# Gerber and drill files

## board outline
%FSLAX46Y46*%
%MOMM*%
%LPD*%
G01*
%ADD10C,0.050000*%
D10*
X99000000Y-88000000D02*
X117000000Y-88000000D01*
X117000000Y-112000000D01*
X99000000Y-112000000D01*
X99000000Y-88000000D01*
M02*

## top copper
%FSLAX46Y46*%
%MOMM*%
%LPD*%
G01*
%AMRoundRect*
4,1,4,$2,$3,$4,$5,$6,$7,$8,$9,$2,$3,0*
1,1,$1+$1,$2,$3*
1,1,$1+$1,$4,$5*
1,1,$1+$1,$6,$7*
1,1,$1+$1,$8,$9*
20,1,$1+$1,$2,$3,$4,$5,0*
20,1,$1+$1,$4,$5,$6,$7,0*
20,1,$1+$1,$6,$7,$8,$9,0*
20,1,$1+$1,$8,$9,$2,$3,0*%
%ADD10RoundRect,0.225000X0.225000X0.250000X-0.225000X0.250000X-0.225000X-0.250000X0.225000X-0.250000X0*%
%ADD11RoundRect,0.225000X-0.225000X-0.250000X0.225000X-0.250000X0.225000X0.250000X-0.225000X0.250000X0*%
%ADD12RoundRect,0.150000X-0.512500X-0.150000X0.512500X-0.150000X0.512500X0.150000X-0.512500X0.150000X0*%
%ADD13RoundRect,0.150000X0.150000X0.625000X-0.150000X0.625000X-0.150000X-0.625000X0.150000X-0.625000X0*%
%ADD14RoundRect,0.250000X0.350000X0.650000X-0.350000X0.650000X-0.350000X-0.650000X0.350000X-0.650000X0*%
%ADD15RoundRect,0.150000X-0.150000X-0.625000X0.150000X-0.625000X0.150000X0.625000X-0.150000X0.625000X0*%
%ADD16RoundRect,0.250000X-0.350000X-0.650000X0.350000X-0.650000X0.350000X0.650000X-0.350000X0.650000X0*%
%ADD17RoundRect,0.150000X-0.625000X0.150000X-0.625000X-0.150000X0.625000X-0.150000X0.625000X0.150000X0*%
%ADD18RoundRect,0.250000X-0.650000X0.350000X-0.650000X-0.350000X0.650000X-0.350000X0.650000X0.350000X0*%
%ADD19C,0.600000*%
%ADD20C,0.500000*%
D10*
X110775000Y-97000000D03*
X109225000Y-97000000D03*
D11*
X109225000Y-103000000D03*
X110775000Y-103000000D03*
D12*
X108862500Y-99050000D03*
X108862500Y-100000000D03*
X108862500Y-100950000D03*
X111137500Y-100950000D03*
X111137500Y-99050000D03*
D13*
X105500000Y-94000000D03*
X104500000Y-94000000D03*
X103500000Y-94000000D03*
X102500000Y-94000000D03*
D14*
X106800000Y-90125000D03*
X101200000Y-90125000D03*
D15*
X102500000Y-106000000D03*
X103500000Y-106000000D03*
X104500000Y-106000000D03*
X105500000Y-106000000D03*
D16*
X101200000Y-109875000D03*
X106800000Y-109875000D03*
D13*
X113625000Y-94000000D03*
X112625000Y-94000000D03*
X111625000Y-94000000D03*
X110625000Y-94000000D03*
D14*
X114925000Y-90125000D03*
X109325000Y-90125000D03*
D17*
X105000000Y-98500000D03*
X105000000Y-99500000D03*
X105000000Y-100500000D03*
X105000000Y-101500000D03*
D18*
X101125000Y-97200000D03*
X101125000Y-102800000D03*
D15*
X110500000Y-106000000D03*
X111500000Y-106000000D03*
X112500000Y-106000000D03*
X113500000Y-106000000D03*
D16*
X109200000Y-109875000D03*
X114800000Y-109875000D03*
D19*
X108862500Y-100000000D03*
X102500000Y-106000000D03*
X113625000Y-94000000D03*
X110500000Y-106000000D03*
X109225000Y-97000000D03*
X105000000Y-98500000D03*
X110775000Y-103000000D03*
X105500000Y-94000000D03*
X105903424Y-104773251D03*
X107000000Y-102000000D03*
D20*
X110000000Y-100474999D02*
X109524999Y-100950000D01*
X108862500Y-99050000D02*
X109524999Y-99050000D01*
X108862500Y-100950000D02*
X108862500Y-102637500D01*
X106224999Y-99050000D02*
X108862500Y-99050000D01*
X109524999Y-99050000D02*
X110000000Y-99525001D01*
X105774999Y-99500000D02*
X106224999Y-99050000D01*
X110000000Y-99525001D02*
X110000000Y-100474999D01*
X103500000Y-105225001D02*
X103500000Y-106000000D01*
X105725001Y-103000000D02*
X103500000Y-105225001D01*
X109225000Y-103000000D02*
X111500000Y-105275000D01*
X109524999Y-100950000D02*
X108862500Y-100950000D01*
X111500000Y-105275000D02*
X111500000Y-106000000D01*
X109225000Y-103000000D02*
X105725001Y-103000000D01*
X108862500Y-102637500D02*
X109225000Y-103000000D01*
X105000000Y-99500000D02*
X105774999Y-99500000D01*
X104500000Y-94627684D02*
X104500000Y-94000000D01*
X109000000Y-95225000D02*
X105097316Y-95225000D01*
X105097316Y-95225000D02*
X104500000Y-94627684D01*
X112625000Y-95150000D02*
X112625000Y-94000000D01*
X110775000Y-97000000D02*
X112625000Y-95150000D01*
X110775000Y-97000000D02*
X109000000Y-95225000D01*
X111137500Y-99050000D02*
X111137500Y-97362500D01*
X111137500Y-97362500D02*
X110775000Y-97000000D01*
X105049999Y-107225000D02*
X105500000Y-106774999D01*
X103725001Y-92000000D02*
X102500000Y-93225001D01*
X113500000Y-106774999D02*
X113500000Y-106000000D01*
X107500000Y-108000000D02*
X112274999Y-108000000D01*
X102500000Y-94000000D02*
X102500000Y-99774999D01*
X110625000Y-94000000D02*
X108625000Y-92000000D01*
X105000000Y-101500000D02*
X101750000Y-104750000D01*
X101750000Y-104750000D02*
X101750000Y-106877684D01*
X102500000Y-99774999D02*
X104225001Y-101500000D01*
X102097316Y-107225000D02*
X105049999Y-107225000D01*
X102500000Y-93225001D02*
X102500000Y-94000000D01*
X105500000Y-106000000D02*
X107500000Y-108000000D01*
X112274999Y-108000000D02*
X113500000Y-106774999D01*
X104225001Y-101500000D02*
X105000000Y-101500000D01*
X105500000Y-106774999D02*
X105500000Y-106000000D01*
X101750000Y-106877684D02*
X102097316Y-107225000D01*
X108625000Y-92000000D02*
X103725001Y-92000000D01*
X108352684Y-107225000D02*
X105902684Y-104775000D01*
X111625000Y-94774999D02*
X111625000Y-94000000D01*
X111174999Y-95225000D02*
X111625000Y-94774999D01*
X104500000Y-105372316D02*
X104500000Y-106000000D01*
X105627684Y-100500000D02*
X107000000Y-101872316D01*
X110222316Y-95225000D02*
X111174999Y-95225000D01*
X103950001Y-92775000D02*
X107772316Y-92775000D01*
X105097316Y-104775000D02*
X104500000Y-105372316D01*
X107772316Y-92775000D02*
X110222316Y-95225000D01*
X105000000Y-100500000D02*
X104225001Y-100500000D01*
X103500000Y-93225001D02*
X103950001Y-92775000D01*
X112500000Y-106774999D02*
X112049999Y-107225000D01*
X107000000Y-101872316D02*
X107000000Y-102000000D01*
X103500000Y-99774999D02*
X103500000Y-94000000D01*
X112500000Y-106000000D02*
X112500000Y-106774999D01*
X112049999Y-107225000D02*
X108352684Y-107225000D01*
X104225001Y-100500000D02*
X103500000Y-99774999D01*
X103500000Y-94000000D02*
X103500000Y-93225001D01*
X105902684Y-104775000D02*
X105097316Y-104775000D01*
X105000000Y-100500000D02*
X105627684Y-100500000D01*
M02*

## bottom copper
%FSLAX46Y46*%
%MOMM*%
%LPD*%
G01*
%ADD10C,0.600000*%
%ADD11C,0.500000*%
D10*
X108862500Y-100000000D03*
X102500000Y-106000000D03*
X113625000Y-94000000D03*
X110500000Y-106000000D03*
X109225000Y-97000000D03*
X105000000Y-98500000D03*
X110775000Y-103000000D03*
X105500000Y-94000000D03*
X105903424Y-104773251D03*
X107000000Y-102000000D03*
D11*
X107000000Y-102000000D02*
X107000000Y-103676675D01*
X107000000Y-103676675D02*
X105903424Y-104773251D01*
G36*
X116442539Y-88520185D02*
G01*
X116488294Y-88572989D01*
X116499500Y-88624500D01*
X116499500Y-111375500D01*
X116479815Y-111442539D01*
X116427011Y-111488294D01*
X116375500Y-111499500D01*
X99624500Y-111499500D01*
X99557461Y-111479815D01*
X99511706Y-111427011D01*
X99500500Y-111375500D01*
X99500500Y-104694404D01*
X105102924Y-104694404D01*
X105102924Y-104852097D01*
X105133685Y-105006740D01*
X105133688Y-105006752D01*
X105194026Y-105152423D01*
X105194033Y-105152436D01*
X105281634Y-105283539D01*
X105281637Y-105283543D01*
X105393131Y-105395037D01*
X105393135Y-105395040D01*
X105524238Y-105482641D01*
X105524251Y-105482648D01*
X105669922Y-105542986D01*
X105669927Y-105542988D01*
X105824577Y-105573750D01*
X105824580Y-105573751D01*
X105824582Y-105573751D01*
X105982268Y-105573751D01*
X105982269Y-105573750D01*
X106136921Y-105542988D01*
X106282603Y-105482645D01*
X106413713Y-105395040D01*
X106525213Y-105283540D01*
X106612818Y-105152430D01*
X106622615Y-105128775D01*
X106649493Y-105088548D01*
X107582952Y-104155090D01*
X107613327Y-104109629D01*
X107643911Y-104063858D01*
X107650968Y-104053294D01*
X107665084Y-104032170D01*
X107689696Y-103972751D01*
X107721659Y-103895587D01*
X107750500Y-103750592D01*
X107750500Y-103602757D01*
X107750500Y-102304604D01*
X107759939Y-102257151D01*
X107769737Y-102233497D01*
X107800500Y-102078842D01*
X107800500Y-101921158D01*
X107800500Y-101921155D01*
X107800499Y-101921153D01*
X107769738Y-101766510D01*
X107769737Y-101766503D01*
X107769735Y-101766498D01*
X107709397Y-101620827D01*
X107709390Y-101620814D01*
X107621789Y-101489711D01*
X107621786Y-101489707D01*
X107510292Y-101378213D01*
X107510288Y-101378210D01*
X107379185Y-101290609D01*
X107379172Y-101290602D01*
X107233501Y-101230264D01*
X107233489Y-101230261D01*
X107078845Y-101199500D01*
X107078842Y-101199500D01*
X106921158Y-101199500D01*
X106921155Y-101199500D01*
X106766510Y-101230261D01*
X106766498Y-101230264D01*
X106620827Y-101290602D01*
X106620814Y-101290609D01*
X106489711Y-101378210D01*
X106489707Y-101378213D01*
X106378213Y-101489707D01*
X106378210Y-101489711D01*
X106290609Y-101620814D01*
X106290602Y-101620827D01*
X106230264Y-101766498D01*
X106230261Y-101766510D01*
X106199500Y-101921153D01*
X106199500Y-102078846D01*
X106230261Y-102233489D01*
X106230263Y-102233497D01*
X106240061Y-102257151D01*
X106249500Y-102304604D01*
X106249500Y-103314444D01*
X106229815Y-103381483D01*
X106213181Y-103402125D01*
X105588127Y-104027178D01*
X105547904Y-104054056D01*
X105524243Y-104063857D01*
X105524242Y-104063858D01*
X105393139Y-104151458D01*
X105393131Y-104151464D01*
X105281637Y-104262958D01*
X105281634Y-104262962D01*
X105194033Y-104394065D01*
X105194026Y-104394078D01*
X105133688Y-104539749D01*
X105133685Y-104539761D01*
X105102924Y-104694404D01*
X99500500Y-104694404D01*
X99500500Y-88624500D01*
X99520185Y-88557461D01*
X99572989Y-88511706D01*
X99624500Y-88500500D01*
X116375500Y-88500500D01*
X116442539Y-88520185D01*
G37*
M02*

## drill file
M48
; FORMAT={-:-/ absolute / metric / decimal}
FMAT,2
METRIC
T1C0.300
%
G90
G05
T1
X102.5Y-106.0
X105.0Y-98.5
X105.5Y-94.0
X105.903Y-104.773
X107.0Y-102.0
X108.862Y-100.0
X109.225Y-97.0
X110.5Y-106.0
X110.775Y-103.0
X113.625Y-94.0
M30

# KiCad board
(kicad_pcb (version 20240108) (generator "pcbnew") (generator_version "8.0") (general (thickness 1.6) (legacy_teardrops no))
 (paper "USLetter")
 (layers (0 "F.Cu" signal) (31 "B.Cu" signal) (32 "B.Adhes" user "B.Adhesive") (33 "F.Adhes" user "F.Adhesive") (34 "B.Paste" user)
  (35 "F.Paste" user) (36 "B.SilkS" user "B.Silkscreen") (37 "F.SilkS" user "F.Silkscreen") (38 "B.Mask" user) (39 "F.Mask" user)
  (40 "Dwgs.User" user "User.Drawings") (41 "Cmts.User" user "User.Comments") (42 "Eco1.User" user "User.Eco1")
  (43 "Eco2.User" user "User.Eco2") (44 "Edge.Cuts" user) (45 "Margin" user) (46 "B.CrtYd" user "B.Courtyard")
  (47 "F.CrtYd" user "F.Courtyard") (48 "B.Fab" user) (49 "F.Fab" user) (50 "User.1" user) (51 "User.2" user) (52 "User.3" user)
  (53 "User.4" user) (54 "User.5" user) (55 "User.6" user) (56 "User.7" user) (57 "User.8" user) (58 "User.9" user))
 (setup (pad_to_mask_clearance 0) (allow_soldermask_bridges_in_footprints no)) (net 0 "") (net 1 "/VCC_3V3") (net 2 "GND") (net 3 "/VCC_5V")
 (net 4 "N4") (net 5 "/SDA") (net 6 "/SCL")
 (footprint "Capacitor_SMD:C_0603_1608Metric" (layer "F.Cu") (at 110 97 180)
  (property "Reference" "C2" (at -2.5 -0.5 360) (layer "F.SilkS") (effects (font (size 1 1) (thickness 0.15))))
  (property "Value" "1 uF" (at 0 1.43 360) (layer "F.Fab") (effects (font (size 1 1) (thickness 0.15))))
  (pad "1" smd roundrect (at -0.775 0 180) (size 0.9 0.95) (layers "F.Cu" "F.Paste" "F.Mask") (roundrect_rratio 0.25) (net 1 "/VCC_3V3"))
  (pad "2" smd roundrect (at 0.775 0 180) (size 0.9 0.95) (layers "F.Cu" "F.Paste" "F.Mask") (roundrect_rratio 0.25) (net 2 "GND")))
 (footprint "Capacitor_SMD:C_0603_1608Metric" (layer "F.Cu") (at 110 103)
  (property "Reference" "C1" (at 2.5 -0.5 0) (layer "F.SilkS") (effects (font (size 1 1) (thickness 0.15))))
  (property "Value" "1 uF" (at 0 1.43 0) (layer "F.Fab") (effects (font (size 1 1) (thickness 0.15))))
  (pad "1" smd roundrect (at -0.775 0) (size 0.9 0.95) (layers "F.Cu" "F.Paste" "F.Mask") (roundrect_rratio 0.25) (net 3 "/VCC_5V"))
  (pad "2" smd roundrect (at 0.775 0) (size 0.9 0.95) (layers "F.Cu" "F.Paste" "F.Mask") (roundrect_rratio 0.25) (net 2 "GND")))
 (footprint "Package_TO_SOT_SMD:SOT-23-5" (layer "F.Cu") (at 110 100)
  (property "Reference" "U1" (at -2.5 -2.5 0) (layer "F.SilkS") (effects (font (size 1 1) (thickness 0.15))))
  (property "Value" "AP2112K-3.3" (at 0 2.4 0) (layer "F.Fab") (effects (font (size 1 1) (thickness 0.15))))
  (pad "1" smd roundrect (at -1.1375 -0.95) (size 1.325 0.6) (layers "F.Cu" "F.Paste" "F.Mask") (roundrect_rratio 0.25) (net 3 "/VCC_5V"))
  (pad "2" smd roundrect (at -1.1375 0) (size 1.325 0.6) (layers "F.Cu" "F.Paste" "F.Mask") (roundrect_rratio 0.25) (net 2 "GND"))
  (pad "3" smd roundrect (at -1.1375 0.95) (size 1.325 0.6) (layers "F.Cu" "F.Paste" "F.Mask") (roundrect_rratio 0.25) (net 3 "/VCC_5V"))
  (pad "4" smd roundrect (at 1.1375 0.95) (size 1.325 0.6) (layers "F.Cu" "F.Paste" "F.Mask") (roundrect_rratio 0.25) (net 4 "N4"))
  (pad "5" smd roundrect (at 1.1375 -0.95) (size 1.325 0.6) (layers "F.Cu" "F.Paste" "F.Mask") (roundrect_rratio 0.25) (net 1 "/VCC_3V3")))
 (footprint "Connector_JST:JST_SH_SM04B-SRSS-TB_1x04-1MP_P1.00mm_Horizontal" (layer "F.Cu") (at 104 92 180)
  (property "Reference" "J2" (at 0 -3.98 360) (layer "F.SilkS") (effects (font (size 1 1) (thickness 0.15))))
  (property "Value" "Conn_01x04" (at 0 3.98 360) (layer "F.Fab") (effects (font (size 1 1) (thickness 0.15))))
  (pad "1" smd roundrect (at -1.5 -2 180) (size 0.6 1.55) (layers "F.Cu" "F.Paste" "F.Mask") (roundrect_rratio 0.25) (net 2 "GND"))
  (pad "2" smd roundrect (at -0.5 -2 180) (size 0.6 1.55) (layers "F.Cu" "F.Paste" "F.Mask") (roundrect_rratio 0.25) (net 1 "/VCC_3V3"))
  (pad "3" smd roundrect (at 0.5 -2 180) (size 0.6 1.55) (layers "F.Cu" "F.Paste" "F.Mask") (roundrect_rratio 0.25) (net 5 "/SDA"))
  (pad "4" smd roundrect (at 1.5 -2 180) (size 0.6 1.55) (layers "F.Cu" "F.Paste" "F.Mask") (roundrect_rratio 0.25) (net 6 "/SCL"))
  (pad "MP" smd roundrect (at -2.8 1.875 180) (size 1.2 1.8) (layers "F.Cu" "F.Paste" "F.Mask") (roundrect_rratio 0.208333))
  (pad "MP" smd roundrect (at 2.8 1.875 180) (size 1.2 1.8) (layers "F.Cu" "F.Paste" "F.Mask") (roundrect_rratio 0.208333)))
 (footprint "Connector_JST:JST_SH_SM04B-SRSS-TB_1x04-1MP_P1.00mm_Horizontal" (layer "F.Cu") (at 104 108)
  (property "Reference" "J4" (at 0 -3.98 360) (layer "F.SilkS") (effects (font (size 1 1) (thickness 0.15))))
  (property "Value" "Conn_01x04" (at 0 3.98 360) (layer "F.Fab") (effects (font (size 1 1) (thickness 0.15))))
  (pad "1" smd roundrect (at -1.5 -2) (size 0.6 1.55) (layers "F.Cu" "F.Paste" "F.Mask") (roundrect_rratio 0.25) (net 2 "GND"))
  (pad "2" smd roundrect (at -0.5 -2) (size 0.6 1.55) (layers "F.Cu" "F.Paste" "F.Mask") (roundrect_rratio 0.25) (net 3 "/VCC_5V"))
  (pad "3" smd roundrect (at 0.5 -2) (size 0.6 1.55) (layers "F.Cu" "F.Paste" "F.Mask") (roundrect_rratio 0.25) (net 5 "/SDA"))
  (pad "4" smd roundrect (at 1.5 -2) (size 0.6 1.55) (layers "F.Cu" "F.Paste" "F.Mask") (roundrect_rratio 0.25) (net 6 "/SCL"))
  (pad "MP" smd roundrect (at -2.8 1.875) (size 1.2 1.8) (layers "F.Cu" "F.Paste" "F.Mask") (roundrect_rratio 0.208333))
  (pad "MP" smd roundrect (at 2.8 1.875) (size 1.2 1.8) (layers "F.Cu" "F.Paste" "F.Mask") (roundrect_rratio 0.208333)))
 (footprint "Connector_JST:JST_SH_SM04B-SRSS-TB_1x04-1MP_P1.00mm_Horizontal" (layer "F.Cu") (at 112.125 92 180)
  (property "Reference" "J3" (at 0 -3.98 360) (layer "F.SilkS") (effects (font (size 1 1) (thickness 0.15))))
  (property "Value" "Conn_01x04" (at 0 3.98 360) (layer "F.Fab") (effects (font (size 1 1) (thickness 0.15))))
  (pad "1" smd roundrect (at -1.5 -2 180) (size 0.6 1.55) (layers "F.Cu" "F.Paste" "F.Mask") (roundrect_rratio 0.25) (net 2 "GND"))
  (pad "2" smd roundrect (at -0.5 -2 180) (size 0.6 1.55) (layers "F.Cu" "F.Paste" "F.Mask") (roundrect_rratio 0.25) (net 1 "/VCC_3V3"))
  (pad "3" smd roundrect (at 0.5 -2 180) (size 0.6 1.55) (layers "F.Cu" "F.Paste" "F.Mask") (roundrect_rratio 0.25) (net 5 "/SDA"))
  (pad "4" smd roundrect (at 1.5 -2 180) (size 0.6 1.55) (layers "F.Cu" "F.Paste" "F.Mask") (roundrect_rratio 0.25) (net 6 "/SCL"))
  (pad "MP" smd roundrect (at -2.8 1.875 180) (size 1.2 1.8) (layers "F.Cu" "F.Paste" "F.Mask") (roundrect_rratio 0.208333))
  (pad "MP" smd roundrect (at 2.8 1.875 180) (size 1.2 1.8) (layers "F.Cu" "F.Paste" "F.Mask") (roundrect_rratio 0.208333)))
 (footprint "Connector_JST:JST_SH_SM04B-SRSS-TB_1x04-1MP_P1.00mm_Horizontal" (layer "F.Cu") (at 103 100 -90)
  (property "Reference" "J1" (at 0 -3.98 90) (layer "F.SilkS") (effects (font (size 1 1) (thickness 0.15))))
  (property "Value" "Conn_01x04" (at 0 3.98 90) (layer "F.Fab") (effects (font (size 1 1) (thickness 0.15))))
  (pad "1" smd roundrect (at -1.5 -2 270) (size 0.6 1.55) (layers "F.Cu" "F.Paste" "F.Mask") (roundrect_rratio 0.25) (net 2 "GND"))
  (pad "2" smd roundrect (at -0.5 -2 270) (size 0.6 1.55) (layers "F.Cu" "F.Paste" "F.Mask") (roundrect_rratio 0.25) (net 3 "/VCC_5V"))
  (pad "3" smd roundrect (at 0.5 -2 270) (size 0.6 1.55) (layers "F.Cu" "F.Paste" "F.Mask") (roundrect_rratio 0.25) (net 5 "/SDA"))
  (pad "4" smd roundrect (at 1.5 -2 270) (size 0.6 1.55) (layers "F.Cu" "F.Paste" "F.Mask") (roundrect_rratio 0.25) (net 6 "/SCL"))
  (pad "MP" smd roundrect (at -2.8 1.875 270) (size 1.2 1.8) (layers "F.Cu" "F.Paste" "F.Mask") (roundrect_rratio 0.208333))
  (pad "MP" smd roundrect (at 2.8 1.875 270) (size 1.2 1.8) (layers "F.Cu" "F.Paste" "F.Mask") (roundrect_rratio 0.208333)))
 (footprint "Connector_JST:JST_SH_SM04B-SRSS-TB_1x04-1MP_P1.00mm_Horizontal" (layer "F.Cu") (at 112 108)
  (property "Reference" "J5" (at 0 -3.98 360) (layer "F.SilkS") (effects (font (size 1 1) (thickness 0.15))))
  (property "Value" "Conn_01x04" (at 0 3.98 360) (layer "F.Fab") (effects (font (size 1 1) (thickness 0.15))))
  (pad "1" smd roundrect (at -1.5 -2) (size 0.6 1.55) (layers "F.Cu" "F.Paste" "F.Mask") (roundrect_rratio 0.25) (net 2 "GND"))
  (pad "2" smd roundrect (at -0.5 -2) (size 0.6 1.55) (layers "F.Cu" "F.Paste" "F.Mask") (roundrect_rratio 0.25) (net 3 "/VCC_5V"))
  (pad "3" smd roundrect (at 0.5 -2) (size 0.6 1.55) (layers "F.Cu" "F.Paste" "F.Mask") (roundrect_rratio 0.25) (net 5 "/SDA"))
  (pad "4" smd roundrect (at 1.5 -2) (size 0.6 1.55) (layers "F.Cu" "F.Paste" "F.Mask") (roundrect_rratio 0.25) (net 6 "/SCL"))
  (pad "MP" smd roundrect (at -2.8 1.875) (size 1.2 1.8) (layers "F.Cu" "F.Paste" "F.Mask") (roundrect_rratio 0.208333))
  (pad "MP" smd roundrect (at 2.8 1.875) (size 1.2 1.8) (layers "F.Cu" "F.Paste" "F.Mask") (roundrect_rratio 0.208333)))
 (gr_rect (start 99 88) (end 117 112) (stroke (width 0.05) (type default)) (fill none) (layer "Edge.Cuts"))
 (via (at 108.8625 100) (size 0.6) (drill 0.3) (layers "F.Cu" "B.Cu") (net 2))
 (via (at 102.5 106) (size 0.6) (drill 0.3) (layers "F.Cu" "B.Cu") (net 2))
 (via (at 113.625 94) (size 0.6) (drill 0.3) (layers "F.Cu" "B.Cu") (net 2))
 (via (at 110.5 106) (size 0.6) (drill 0.3) (layers "F.Cu" "B.Cu") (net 2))
 (via (at 109.225 97) (size 0.6) (drill 0.3) (layers "F.Cu" "B.Cu") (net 2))
 (via (at 105 98.5) (size 0.6) (drill 0.3) (layers "F.Cu" "B.Cu") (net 2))
 (via (at 110.775 103) (size 0.6) (drill 0.3) (layers "F.Cu" "B.Cu") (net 2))
 (via (at 105.5 94) (size 0.6) (drill 0.3) (layers "F.Cu" "B.Cu") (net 2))
 (segment (start 110 100.474999) (end 109.524999 100.95) (width 0.5) (layer "F.Cu") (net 3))
 (segment (start 108.8625 99.05) (end 109.524999 99.05) (width 0.5) (layer "F.Cu") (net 3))
 (segment (start 108.8625 100.95) (end 108.8625 102.6375) (width 0.5) (layer "F.Cu") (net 3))
 (segment (start 106.224999 99.05) (end 108.8625 99.05) (width 0.5) (layer "F.Cu") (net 3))
 (segment (start 109.524999 99.05) (end 110 99.525001) (width 0.5) (layer "F.Cu") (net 3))
 (segment (start 105.774999 99.5) (end 106.224999 99.05) (width 0.5) (layer "F.Cu") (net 3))
 (segment (start 110 99.525001) (end 110 100.474999) (width 0.5) (layer "F.Cu") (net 3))
 (segment (start 103.5 105.225001) (end 103.5 106) (width 0.5) (layer "F.Cu") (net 3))
 (segment (start 105.725001 103) (end 103.5 105.225001) (width 0.5) (layer "F.Cu") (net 3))
 (segment (start 109.225 103) (end 111.5 105.275) (width 0.5) (layer "F.Cu") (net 3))
 (segment (start 109.524999 100.95) (end 108.8625 100.95) (width 0.5) (layer "F.Cu") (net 3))
 (segment (start 111.5 105.275) (end 111.5 106) (width 0.5) (layer "F.Cu") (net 3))
 (segment (start 109.225 103) (end 105.725001 103) (width 0.5) (layer "F.Cu") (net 3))
 (segment (start 108.8625 102.6375) (end 109.225 103) (width 0.5) (layer "F.Cu") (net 3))
 (segment (start 105 99.5) (end 105.774999 99.5) (width 0.5) (layer "F.Cu") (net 3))
 (segment (start 104.5 94.627684) (end 104.5 94) (width 0.5) (layer "F.Cu") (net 1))
 (segment (start 109 95.225) (end 105.097316 95.225) (width 0.5) (layer "F.Cu") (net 1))
 (segment (start 105.097316 95.225) (end 104.5 94.627684) (width 0.5) (layer "F.Cu") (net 1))
 (segment (start 112.625 95.15) (end 112.625 94) (width 0.5) (layer "F.Cu") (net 1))
 (segment (start 110.775 97) (end 112.625 95.15) (width 0.5) (layer "F.Cu") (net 1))
 (segment (start 110.775 97) (end 109 95.225) (width 0.5) (layer "F.Cu") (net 1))
 (segment (start 111.1375 99.05) (end 111.1375 97.3625) (width 0.5) (layer "F.Cu") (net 1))
 (segment (start 111.1375 97.3625) (end 110.775 97) (width 0.5) (layer "F.Cu") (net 1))
 (segment (start 105.049999 107.225) (end 105.5 106.774999) (width 0.5) (layer "F.Cu") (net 6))
 (segment (start 103.725001 92) (end 102.5 93.225001) (width 0.5) (layer "F.Cu") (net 6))
 (segment (start 113.5 106.774999) (end 113.5 106) (width 0.5) (layer "F.Cu") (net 6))
 (segment (start 107.5 108) (end 112.274999 108) (width 0.5) (layer "F.Cu") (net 6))
 (segment (start 102.5 94) (end 102.5 99.774999) (width 0.5) (layer "F.Cu") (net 6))
 (segment (start 110.625 94) (end 108.625 92) (width 0.5) (layer "F.Cu") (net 6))
 (segment (start 105 101.5) (end 101.75 104.75) (width 0.5) (layer "F.Cu") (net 6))
 (segment (start 101.75 104.75) (end 101.75 106.877684) (width 0.5) (layer "F.Cu") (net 6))
 (segment (start 102.5 99.774999) (end 104.225001 101.5) (width 0.5) (layer "F.Cu") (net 6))
 (segment (start 102.097316 107.225) (end 105.049999 107.225) (width 0.5) (layer "F.Cu") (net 6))
 (segment (start 102.5 93.225001) (end 102.5 94) (width 0.5) (layer "F.Cu") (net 6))
 (segment (start 105.5 106) (end 107.5 108) (width 0.5) (layer "F.Cu") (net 6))
 (segment (start 112.274999 108) (end 113.5 106.774999) (width 0.5) (layer "F.Cu") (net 6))
 (segment (start 104.225001 101.5) (end 105 101.5) (width 0.5) (layer "F.Cu") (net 6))
 (segment (start 105.5 106.774999) (end 105.5 106) (width 0.5) (layer "F.Cu") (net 6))
 (segment (start 101.75 106.877684) (end 102.097316 107.225) (width 0.5) (layer "F.Cu") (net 6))
 (segment (start 108.625 92) (end 103.725001 92) (width 0.5) (layer "F.Cu") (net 6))
 (segment (start 108.352684 107.225) (end 105.902684 104.775) (width 0.5) (layer "F.Cu") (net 5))
 (segment (start 111.625 94.774999) (end 111.625 94) (width 0.5) (layer "F.Cu") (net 5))
 (segment (start 111.174999 95.225) (end 111.625 94.774999) (width 0.5) (layer "F.Cu") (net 5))
 (segment (start 104.5 105.372316) (end 104.5 106) (width 0.5) (layer "F.Cu") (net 5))
 (segment (start 105.627684 100.5) (end 107 101.872316) (width 0.5) (layer "F.Cu") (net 5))
 (segment (start 110.222316 95.225) (end 111.174999 95.225) (width 0.5) (layer "F.Cu") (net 5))
 (segment (start 103.950001 92.775) (end 107.772316 92.775) (width 0.5) (layer "F.Cu") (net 5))
 (segment (start 105.097316 104.775) (end 104.5 105.372316) (width 0.5) (layer "F.Cu") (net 5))
 (segment (start 107.772316 92.775) (end 110.222316 95.225) (width 0.5) (layer "F.Cu") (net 5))
 (segment (start 105 100.5) (end 104.225001 100.5) (width 0.5) (layer "F.Cu") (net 5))
 (segment (start 103.5 93.225001) (end 103.950001 92.775) (width 0.5) (layer "F.Cu") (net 5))
 (segment (start 112.5 106.774999) (end 112.049999 107.225) (width 0.5) (layer "F.Cu") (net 5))
 (segment (start 107 101.872316) (end 107 102) (width 0.5) (layer "F.Cu") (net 5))
 (segment (start 103.5 99.774999) (end 103.5 94) (width 0.5) (layer "F.Cu") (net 5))
 (segment (start 112.5 106) (end 112.5 106.774999) (width 0.5) (layer "F.Cu") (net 5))
 (segment (start 112.049999 107.225) (end 108.352684 107.225) (width 0.5) (layer "F.Cu") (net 5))
 (segment (start 104.225001 100.5) (end 103.5 99.774999) (width 0.5) (layer "F.Cu") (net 5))
 (segment (start 103.5 94) (end 103.5 93.225001) (width 0.5) (layer "F.Cu") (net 5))
 (segment (start 105.902684 104.775) (end 105.097316 104.775) (width 0.5) (layer "F.Cu") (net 5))
 (segment (start 105 100.5) (end 105.627684 100.5) (width 0.5) (layer "F.Cu") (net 5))
 (via (at 105.903424 104.773251) (size 0.6) (drill 0.3) (layers "F.Cu" "B.Cu") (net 5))
 (via (at 107 102) (size 0.6) (drill 0.3) (layers "F.Cu" "B.Cu") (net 5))
 (segment (start 107 102) (end 107 103.676675) (width 0.5) (layer "B.Cu") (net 5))
 (segment (start 107 103.676675) (end 105.903424 104.773251) (width 0.5) (layer "B.Cu") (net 5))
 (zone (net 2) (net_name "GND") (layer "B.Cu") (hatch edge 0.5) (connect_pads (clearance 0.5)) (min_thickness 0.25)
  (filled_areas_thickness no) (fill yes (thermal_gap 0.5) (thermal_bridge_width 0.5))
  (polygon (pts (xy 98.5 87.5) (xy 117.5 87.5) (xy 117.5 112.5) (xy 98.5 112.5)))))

